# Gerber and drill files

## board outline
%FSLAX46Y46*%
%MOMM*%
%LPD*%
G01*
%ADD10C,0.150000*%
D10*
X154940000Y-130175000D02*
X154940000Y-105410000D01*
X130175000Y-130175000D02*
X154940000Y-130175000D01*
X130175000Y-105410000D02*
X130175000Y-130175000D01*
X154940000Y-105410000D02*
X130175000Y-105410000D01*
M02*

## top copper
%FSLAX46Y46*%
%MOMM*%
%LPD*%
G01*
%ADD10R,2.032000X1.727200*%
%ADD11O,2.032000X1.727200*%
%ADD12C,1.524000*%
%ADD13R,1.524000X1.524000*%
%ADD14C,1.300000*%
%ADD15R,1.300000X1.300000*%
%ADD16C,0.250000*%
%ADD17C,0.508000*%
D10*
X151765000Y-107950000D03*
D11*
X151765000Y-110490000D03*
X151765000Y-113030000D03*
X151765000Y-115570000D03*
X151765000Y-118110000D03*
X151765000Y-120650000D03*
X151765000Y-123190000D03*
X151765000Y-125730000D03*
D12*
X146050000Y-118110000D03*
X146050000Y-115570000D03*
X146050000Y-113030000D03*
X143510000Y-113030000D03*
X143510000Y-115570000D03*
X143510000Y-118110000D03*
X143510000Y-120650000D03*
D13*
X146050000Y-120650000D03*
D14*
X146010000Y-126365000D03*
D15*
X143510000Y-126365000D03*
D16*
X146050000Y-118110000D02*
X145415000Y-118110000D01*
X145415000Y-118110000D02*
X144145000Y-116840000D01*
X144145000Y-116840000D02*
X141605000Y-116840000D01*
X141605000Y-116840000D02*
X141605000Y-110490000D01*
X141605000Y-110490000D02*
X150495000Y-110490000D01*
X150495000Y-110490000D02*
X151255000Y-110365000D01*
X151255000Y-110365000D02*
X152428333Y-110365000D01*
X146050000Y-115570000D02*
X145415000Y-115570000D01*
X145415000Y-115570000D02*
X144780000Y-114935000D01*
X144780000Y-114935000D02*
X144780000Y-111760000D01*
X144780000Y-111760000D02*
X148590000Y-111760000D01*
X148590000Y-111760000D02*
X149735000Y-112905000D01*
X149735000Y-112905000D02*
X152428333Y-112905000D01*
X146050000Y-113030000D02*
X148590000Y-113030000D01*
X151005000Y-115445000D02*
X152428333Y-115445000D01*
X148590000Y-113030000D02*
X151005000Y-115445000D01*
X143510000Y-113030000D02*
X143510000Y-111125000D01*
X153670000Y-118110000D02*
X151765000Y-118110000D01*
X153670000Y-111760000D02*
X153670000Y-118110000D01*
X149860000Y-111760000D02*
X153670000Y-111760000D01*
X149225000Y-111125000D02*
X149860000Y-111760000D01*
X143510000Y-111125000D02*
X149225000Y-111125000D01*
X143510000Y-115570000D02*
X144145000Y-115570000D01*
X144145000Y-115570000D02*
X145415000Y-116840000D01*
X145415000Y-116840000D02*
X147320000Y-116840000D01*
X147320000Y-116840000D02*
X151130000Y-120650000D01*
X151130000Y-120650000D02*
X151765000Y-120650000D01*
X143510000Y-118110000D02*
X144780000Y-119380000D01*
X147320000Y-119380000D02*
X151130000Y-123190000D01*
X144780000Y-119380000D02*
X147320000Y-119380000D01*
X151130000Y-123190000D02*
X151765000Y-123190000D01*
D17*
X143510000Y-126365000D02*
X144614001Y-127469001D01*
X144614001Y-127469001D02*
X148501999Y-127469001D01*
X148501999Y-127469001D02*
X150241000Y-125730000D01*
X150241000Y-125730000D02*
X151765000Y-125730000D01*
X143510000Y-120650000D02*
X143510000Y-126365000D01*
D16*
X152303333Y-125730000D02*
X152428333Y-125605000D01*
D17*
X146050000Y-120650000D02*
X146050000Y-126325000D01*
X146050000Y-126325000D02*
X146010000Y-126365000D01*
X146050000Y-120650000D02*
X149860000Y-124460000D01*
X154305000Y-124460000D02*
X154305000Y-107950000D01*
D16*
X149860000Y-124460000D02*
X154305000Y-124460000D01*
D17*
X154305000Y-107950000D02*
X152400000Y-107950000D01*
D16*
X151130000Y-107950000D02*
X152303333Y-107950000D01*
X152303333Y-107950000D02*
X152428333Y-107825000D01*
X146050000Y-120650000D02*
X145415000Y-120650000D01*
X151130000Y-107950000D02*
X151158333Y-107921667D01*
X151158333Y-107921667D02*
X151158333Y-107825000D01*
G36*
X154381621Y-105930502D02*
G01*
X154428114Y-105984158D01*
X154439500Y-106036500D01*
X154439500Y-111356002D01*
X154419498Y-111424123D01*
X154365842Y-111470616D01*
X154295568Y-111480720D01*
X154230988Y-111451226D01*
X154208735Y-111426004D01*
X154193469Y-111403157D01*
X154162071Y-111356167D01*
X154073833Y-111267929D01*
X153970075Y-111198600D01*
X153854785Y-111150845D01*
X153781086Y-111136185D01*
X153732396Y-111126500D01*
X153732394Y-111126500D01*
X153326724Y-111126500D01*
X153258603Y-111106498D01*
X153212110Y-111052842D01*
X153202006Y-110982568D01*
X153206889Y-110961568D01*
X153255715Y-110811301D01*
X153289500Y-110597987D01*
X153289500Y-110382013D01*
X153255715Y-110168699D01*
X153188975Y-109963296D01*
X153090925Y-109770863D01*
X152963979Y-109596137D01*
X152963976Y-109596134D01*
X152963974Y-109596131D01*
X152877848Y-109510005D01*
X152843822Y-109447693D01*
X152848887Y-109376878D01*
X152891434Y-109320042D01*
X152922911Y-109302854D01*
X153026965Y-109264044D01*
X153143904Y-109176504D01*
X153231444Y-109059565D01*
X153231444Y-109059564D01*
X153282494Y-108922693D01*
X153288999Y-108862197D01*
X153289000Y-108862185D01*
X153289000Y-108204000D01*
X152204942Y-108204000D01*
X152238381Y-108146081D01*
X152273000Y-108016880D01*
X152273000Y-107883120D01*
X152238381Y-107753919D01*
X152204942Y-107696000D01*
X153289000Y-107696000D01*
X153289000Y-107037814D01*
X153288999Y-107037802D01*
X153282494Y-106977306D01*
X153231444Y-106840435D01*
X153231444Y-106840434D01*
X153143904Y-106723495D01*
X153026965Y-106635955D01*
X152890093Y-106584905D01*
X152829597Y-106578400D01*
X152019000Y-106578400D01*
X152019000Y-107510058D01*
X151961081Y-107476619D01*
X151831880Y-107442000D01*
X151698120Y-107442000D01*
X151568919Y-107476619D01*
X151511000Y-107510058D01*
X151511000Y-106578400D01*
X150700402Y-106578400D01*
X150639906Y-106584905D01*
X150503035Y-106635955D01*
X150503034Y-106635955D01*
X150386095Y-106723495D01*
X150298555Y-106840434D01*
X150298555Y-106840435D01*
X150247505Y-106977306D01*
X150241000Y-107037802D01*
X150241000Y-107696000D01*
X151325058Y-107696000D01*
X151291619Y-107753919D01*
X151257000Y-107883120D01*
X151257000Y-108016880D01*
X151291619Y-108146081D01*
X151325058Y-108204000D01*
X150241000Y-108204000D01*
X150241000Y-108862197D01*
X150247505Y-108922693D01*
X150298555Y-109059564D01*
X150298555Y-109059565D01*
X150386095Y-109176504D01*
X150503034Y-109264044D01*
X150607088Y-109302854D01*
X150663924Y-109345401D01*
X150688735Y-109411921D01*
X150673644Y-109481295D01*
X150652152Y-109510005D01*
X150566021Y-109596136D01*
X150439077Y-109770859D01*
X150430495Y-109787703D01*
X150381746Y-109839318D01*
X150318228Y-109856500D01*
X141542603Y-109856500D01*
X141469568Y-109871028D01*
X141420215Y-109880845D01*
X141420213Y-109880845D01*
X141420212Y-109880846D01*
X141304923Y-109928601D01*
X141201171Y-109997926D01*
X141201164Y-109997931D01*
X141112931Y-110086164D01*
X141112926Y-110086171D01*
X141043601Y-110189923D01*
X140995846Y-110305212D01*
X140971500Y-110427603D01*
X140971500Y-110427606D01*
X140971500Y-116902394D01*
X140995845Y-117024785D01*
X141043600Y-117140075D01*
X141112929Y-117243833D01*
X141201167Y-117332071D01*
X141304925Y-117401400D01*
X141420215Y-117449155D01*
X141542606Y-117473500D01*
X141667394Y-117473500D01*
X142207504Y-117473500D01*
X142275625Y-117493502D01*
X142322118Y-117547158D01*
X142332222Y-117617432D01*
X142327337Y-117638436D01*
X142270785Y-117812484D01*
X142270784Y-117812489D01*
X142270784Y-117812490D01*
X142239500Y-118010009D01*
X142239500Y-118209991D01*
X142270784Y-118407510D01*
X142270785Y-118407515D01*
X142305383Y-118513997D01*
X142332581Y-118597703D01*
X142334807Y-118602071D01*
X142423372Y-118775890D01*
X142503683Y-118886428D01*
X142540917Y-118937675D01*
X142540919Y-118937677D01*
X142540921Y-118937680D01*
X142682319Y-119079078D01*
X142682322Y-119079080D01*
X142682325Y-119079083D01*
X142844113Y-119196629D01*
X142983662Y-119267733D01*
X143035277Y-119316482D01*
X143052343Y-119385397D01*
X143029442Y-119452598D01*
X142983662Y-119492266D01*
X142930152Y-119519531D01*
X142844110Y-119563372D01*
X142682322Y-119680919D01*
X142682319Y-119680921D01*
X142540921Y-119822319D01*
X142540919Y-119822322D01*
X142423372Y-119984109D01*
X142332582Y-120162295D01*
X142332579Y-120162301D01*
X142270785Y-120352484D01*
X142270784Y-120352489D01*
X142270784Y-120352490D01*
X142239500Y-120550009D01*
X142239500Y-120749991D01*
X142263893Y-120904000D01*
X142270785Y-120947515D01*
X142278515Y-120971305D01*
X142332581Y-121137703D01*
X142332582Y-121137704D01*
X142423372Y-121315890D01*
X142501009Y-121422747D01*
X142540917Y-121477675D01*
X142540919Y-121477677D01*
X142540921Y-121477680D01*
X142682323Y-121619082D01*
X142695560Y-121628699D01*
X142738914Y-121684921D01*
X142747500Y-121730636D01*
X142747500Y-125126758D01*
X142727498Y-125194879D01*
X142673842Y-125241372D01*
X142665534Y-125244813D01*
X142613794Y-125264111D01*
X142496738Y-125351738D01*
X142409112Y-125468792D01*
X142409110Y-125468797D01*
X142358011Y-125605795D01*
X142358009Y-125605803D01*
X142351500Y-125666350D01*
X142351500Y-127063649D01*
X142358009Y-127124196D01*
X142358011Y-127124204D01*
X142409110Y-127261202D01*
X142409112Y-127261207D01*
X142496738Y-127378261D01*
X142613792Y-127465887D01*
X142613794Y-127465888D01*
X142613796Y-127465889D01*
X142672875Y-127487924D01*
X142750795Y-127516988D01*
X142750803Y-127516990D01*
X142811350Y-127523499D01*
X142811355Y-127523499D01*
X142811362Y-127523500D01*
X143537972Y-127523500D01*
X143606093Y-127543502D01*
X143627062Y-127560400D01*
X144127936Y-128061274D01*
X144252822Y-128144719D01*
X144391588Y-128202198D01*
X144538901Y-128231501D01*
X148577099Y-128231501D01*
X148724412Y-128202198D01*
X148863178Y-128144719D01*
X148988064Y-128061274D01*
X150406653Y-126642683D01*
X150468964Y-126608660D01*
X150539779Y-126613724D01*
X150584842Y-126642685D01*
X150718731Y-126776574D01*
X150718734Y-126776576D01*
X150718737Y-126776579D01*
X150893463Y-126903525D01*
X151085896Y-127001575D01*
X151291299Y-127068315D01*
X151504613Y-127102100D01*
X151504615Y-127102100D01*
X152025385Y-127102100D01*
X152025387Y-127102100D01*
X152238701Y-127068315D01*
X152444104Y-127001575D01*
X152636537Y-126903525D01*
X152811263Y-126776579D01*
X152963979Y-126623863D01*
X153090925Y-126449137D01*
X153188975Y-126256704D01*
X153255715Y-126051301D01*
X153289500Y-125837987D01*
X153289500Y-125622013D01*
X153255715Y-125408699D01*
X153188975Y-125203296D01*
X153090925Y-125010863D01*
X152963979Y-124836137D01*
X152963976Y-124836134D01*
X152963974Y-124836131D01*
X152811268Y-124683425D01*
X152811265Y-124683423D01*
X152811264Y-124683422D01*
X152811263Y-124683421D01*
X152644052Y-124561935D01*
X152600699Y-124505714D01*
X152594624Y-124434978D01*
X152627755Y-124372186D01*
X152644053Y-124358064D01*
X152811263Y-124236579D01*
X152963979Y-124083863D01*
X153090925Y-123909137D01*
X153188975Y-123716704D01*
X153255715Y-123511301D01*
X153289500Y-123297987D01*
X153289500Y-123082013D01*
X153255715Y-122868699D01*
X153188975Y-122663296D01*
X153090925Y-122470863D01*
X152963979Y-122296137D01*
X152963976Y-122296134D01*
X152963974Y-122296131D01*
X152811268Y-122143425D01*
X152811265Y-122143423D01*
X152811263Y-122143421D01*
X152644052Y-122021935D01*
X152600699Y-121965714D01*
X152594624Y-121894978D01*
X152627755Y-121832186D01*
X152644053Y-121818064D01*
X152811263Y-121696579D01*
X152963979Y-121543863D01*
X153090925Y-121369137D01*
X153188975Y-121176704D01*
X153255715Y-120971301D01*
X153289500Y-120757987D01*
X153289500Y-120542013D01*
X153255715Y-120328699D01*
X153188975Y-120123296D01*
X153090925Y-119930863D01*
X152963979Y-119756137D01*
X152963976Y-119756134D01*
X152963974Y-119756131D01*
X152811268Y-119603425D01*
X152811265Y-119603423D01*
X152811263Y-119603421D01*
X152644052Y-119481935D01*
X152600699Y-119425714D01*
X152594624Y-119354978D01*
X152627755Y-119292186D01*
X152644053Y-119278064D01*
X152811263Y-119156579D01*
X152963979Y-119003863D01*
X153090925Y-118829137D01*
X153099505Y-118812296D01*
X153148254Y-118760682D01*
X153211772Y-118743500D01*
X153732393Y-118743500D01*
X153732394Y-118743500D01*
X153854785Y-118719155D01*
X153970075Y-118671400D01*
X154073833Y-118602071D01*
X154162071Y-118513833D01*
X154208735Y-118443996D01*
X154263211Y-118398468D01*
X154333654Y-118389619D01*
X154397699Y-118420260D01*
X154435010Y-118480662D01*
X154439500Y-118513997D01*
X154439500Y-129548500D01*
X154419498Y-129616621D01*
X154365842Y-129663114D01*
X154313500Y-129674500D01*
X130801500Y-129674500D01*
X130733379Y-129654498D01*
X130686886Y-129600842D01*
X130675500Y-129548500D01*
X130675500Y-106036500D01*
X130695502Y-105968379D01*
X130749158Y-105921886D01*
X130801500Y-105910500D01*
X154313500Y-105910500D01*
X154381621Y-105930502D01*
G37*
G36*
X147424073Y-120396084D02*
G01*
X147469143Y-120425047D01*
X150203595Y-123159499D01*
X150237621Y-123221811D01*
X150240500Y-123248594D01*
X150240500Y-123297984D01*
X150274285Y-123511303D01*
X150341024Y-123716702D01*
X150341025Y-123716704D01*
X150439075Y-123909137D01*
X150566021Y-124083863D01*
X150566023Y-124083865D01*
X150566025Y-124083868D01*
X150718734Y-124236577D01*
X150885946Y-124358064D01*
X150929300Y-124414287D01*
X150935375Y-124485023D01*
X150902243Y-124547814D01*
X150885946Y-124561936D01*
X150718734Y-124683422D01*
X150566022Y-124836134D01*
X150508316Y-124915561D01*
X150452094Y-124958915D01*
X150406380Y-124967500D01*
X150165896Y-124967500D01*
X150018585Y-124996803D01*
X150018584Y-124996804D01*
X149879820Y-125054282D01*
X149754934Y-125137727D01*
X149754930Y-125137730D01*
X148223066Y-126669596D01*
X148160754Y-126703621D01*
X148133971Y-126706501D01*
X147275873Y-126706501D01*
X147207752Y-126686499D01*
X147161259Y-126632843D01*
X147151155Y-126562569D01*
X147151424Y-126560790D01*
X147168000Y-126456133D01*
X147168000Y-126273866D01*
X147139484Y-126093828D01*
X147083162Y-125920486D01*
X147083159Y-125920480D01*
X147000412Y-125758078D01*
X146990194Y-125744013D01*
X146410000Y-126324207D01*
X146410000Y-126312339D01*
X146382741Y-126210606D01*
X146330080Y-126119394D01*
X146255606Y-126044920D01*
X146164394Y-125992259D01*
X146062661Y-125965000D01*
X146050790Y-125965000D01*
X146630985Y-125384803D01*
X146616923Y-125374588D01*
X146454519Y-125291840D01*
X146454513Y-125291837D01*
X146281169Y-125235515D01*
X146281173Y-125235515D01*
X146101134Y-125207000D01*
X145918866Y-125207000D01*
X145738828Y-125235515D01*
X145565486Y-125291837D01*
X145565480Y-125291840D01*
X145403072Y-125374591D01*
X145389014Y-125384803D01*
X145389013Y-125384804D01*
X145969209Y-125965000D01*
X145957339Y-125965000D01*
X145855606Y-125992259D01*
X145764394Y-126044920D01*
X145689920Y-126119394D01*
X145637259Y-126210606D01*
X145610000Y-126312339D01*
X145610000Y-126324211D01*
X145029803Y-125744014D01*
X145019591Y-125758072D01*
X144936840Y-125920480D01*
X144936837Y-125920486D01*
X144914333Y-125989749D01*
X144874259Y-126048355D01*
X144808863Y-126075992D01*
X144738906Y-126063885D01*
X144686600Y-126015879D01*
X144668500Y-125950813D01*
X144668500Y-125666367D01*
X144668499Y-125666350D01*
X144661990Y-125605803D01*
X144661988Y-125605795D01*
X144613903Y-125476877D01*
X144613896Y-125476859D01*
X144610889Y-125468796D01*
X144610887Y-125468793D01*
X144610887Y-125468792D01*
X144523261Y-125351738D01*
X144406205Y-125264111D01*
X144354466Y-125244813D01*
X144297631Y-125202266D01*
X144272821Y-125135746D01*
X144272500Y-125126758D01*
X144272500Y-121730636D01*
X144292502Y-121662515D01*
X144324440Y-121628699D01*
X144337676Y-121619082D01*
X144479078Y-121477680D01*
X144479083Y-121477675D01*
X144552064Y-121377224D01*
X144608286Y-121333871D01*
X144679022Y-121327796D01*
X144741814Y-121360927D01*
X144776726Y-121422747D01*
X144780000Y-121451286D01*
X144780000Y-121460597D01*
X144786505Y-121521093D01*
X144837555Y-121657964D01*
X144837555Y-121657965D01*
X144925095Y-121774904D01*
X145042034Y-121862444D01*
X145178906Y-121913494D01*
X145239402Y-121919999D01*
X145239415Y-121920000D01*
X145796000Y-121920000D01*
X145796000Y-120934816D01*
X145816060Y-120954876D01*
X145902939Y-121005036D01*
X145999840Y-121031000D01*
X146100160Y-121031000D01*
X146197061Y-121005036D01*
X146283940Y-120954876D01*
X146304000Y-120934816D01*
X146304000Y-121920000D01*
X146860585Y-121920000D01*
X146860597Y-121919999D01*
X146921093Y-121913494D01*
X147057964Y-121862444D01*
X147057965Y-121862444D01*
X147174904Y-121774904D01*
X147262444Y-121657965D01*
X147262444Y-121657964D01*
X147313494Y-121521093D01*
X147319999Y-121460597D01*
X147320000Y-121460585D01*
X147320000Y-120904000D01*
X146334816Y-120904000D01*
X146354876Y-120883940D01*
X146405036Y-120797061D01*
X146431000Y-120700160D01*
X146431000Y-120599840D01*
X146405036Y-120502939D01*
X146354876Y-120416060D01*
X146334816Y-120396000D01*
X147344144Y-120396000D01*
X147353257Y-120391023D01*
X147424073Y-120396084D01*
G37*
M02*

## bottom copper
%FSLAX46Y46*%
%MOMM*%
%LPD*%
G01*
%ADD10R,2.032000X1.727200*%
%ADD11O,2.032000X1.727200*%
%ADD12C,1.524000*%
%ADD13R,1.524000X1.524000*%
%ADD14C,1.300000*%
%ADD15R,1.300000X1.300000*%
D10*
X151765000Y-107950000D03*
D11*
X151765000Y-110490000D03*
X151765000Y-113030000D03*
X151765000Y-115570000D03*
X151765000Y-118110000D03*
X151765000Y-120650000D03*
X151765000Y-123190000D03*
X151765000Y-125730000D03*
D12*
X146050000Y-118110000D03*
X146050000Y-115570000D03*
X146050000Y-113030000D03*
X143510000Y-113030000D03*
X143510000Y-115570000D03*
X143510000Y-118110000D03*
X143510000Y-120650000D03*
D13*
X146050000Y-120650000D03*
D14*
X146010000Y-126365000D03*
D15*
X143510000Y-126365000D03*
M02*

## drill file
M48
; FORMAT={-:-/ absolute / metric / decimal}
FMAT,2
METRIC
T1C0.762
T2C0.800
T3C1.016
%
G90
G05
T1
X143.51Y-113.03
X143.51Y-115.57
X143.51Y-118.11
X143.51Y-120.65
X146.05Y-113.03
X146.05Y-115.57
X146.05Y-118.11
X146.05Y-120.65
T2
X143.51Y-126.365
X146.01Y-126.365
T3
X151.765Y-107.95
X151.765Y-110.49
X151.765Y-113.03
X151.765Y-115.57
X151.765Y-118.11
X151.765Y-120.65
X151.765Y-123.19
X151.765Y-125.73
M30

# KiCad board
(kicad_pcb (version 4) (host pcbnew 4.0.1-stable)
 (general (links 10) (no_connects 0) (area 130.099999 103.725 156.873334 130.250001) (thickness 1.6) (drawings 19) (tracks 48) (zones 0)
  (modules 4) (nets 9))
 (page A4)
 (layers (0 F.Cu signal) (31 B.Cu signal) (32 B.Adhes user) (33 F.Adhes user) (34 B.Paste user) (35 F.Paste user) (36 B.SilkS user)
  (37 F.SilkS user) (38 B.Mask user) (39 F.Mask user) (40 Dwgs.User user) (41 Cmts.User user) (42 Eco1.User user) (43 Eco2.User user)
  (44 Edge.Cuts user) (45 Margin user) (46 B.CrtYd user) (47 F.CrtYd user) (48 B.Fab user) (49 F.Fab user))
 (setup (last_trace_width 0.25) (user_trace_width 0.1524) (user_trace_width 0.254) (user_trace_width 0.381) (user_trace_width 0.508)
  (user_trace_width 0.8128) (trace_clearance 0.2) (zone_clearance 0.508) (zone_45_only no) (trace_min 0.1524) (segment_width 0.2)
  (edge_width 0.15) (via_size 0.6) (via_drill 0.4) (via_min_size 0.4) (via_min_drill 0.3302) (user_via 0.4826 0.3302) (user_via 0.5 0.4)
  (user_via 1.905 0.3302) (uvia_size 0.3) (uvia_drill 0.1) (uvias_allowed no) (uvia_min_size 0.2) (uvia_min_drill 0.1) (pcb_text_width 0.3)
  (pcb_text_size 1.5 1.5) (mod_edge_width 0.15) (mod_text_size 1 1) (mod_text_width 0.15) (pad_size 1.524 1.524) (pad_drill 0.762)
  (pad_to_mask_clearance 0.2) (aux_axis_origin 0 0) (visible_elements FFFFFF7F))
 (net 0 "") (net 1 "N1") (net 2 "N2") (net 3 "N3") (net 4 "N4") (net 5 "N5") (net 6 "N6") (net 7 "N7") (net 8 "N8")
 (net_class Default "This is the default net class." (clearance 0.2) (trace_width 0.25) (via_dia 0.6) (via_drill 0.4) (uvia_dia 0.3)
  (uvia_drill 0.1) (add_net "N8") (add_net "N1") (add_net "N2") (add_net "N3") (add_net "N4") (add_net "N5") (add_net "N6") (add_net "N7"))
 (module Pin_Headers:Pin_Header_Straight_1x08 (layer F.Cu) (at 151.765 107.95)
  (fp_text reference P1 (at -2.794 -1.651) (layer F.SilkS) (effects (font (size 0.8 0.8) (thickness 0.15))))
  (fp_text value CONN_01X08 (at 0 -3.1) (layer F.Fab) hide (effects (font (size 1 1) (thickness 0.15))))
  (pad 1 thru_hole rect (at 0 0) (size 2.032 1.7272) (drill 1.016) (layers *.Cu *.Mask F.SilkS) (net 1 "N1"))
  (pad 2 thru_hole oval (at 0 2.54) (size 2.032 1.7272) (drill 1.016) (layers *.Cu *.Mask F.SilkS) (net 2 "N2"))
  (pad 3 thru_hole oval (at 0 5.08) (size 2.032 1.7272) (drill 1.016) (layers *.Cu *.Mask F.SilkS) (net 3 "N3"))
  (pad 4 thru_hole oval (at 0 7.62) (size 2.032 1.7272) (drill 1.016) (layers *.Cu *.Mask F.SilkS) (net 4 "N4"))
  (pad 5 thru_hole oval (at 0 10.16) (size 2.032 1.7272) (drill 1.016) (layers *.Cu *.Mask F.SilkS) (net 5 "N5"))
  (pad 6 thru_hole oval (at 0 12.7) (size 2.032 1.7272) (drill 1.016) (layers *.Cu *.Mask F.SilkS) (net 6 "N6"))
  (pad 7 thru_hole oval (at 0 15.24) (size 2.032 1.7272) (drill 1.016) (layers *.Cu *.Mask F.SilkS) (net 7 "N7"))
  (pad 8 thru_hole oval (at 0 17.78) (size 2.032 1.7272) (drill 1.016) (layers *.Cu *.Mask F.SilkS) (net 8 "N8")))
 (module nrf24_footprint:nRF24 (layer F.Cu) (at 138.43 120.65)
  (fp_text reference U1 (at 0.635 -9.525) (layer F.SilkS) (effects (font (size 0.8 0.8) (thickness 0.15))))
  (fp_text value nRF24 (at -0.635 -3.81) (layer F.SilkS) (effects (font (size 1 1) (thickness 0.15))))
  (pad 1 thru_hole circle (at 7.62 -2.54) (size 1.524 1.524) (drill 0.762) (layers *.Cu *.Mask F.SilkS) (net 2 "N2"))
  (pad 2 thru_hole circle (at 7.62 -5.08) (size 1.524 1.524) (drill 0.762) (layers *.Cu *.Mask F.SilkS) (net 3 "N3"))
  (pad 3 thru_hole circle (at 7.62 -7.62) (size 1.524 1.524) (drill 0.762) (layers *.Cu *.Mask F.SilkS) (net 4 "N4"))
  (pad 4 thru_hole circle (at 5.08 -7.62) (size 1.524 1.524) (drill 0.762) (layers *.Cu *.Mask F.SilkS) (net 5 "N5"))
  (pad 5 thru_hole circle (at 5.08 -5.08) (size 1.524 1.524) (drill 0.762) (layers *.Cu *.Mask F.SilkS) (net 6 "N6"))
  (pad 6 thru_hole circle (at 5.08 -2.54) (size 1.524 1.524) (drill 0.762) (layers *.Cu *.Mask F.SilkS) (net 7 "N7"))
  (pad 7 thru_hole circle (at 5.08 0) (size 1.524 1.524) (drill 0.762) (layers *.Cu *.Mask F.SilkS) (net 8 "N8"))
  (pad 0 thru_hole rect (at 7.62 0) (size 1.524 1.524) (drill 0.762) (layers *.Cu *.Mask F.SilkS) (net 1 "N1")))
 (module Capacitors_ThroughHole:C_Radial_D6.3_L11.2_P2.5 (layer F.Cu) (at 143.51 126.365)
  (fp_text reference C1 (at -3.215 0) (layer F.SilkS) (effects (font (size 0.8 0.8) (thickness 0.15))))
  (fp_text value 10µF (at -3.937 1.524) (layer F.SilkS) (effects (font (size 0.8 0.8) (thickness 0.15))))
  (pad 2 thru_hole circle (at 2.5 0) (size 1.3 1.3) (drill 0.8) (layers *.Cu *.Mask F.SilkS) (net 1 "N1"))
  (pad 1 thru_hole rect (at 0 0) (size 1.3 1.3) (drill 0.8) (layers *.Cu *.Mask F.SilkS) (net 8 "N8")))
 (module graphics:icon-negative (layer F.Cu) (at 134.62 126.238)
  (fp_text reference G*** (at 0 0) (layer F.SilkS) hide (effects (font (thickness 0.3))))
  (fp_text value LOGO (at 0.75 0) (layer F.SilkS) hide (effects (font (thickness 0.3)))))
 (gr_line (start 154.94 130.175) (end 154.94 105.41) (layer Edge.Cuts) (width 0.15))
 (gr_line (start 130.175 130.175) (end 154.94 130.175) (layer Edge.Cuts) (width 0.15))
 (gr_line (start 130.175 105.41) (end 130.175 130.175) (layer Edge.Cuts) (width 0.15))
 (gr_line (start 154.94 105.41) (end 130.175 105.41) (angle 90) (layer Edge.Cuts) (width 0.15))
 (segment (start 146.05 118.11) (end 145.415 118.11) (width 0.25) (layer F.Cu) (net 2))
 (segment (start 145.415 118.11) (end 144.145 116.84) (width 0.25) (layer F.Cu) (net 2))
 (segment (start 144.145 116.84) (end 141.605 116.84) (width 0.25) (layer F.Cu) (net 2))
 (segment (start 141.605 116.84) (end 141.605 110.49) (width 0.25) (layer F.Cu) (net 2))
 (segment (start 141.605 110.49) (end 150.495 110.49) (width 0.25) (layer F.Cu) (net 2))
 (segment (start 150.495 110.49) (end 151.255 110.365) (width 0.25) (layer F.Cu) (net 2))
 (segment (start 151.255 110.365) (end 152.428333 110.365) (width 0.25) (layer F.Cu) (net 2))
 (segment (start 146.05 115.57) (end 145.415 115.57) (width 0.25) (layer F.Cu) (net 3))
 (segment (start 145.415 115.57) (end 144.78 114.935) (width 0.25) (layer F.Cu) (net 3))
 (segment (start 144.78 114.935) (end 144.78 111.76) (width 0.25) (layer F.Cu) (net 3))
 (segment (start 144.78 111.76) (end 148.59 111.76) (width 0.25) (layer F.Cu) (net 3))
 (segment (start 148.59 111.76) (end 149.735 112.905) (width 0.25) (layer F.Cu) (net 3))
 (segment (start 149.735 112.905) (end 152.428333 112.905) (width 0.25) (layer F.Cu) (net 3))
 (segment (start 146.05 113.03) (end 148.59 113.03) (width 0.25) (layer F.Cu) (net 4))
 (segment (start 151.005 115.445) (end 152.428333 115.445) (width 0.25) (layer F.Cu) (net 4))
 (segment (start 148.59 113.03) (end 151.005 115.445) (width 0.25) (layer F.Cu) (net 4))
 (segment (start 143.51 113.03) (end 143.51 111.125) (width 0.25) (layer F.Cu) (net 5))
 (segment (start 153.67 118.11) (end 151.765 118.11) (width 0.25) (layer F.Cu) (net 5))
 (segment (start 153.67 111.76) (end 153.67 118.11) (width 0.25) (layer F.Cu) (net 5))
 (segment (start 149.86 111.76) (end 153.67 111.76) (width 0.25) (layer F.Cu) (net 5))
 (segment (start 149.225 111.125) (end 149.86 111.76) (width 0.25) (layer F.Cu) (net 5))
 (segment (start 143.51 111.125) (end 149.225 111.125) (width 0.25) (layer F.Cu) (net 5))
 (segment (start 143.51 115.57) (end 144.145 115.57) (width 0.25) (layer F.Cu) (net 6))
 (segment (start 144.145 115.57) (end 145.415 116.84) (width 0.25) (layer F.Cu) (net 6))
 (segment (start 145.415 116.84) (end 147.32 116.84) (width 0.25) (layer F.Cu) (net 6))
 (segment (start 147.32 116.84) (end 151.13 120.65) (width 0.25) (layer F.Cu) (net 6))
 (segment (start 151.13 120.65) (end 151.765 120.65) (width 0.25) (layer F.Cu) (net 6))
 (segment (start 143.51 118.11) (end 144.78 119.38) (width 0.25) (layer F.Cu) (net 7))
 (segment (start 147.32 119.38) (end 151.13 123.19) (width 0.25) (layer F.Cu) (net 7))
 (segment (start 144.78 119.38) (end 147.32 119.38) (width 0.25) (layer F.Cu) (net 7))
 (segment (start 151.13 123.19) (end 151.765 123.19) (width 0.25) (layer F.Cu) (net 7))
 (segment (start 143.51 126.365) (end 144.614001 127.469001) (width 0.508) (layer F.Cu) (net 8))
 (segment (start 144.614001 127.469001) (end 148.501999 127.469001) (width 0.508) (layer F.Cu) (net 8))
 (segment (start 148.501999 127.469001) (end 150.241 125.73) (width 0.508) (layer F.Cu) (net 8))
 (segment (start 150.241 125.73) (end 151.765 125.73) (width 0.508) (layer F.Cu) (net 8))
 (segment (start 143.51 120.65) (end 143.51 126.365) (width 0.508) (layer F.Cu) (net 8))
 (segment (start 152.303333 125.73) (end 152.428333 125.605) (width 0.25) (layer F.Cu) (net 8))
 (segment (start 146.05 120.65) (end 146.05 126.325) (width 0.508) (layer F.Cu) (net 1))
 (segment (start 146.05 126.325) (end 146.01 126.365) (width 0.508) (layer F.Cu) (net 1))
 (segment (start 146.05 120.65) (end 149.86 124.46) (width 0.508) (layer F.Cu) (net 1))
 (segment (start 154.305 124.46) (end 154.305 107.95) (width 0.508) (layer F.Cu) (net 1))
 (segment (start 149.86 124.46) (end 154.305 124.46) (width 0.25) (layer F.Cu) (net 1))
 (segment (start 154.305 107.95) (end 152.4 107.95) (width 0.508) (layer F.Cu) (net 1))
 (segment (start 151.13 107.95) (end 152.303333 107.95) (width 0.25) (layer F.Cu) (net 1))
 (segment (start 152.303333 107.95) (end 152.428333 107.825) (width 0.25) (layer F.Cu) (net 1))
 (segment (start 146.05 120.65) (end 145.415 120.65) (width 0.25) (layer F.Cu) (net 1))
 (segment (start 151.13 107.95) (end 151.158333 107.921667) (width 0.25) (layer F.Cu) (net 1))
 (segment (start 151.158333 107.921667) (end 151.158333 107.825) (width 0.25) (layer F.Cu) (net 1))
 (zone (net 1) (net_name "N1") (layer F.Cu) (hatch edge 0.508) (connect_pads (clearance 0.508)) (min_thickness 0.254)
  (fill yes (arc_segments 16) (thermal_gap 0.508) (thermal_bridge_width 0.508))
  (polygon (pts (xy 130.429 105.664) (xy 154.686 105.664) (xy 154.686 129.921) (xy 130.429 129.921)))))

